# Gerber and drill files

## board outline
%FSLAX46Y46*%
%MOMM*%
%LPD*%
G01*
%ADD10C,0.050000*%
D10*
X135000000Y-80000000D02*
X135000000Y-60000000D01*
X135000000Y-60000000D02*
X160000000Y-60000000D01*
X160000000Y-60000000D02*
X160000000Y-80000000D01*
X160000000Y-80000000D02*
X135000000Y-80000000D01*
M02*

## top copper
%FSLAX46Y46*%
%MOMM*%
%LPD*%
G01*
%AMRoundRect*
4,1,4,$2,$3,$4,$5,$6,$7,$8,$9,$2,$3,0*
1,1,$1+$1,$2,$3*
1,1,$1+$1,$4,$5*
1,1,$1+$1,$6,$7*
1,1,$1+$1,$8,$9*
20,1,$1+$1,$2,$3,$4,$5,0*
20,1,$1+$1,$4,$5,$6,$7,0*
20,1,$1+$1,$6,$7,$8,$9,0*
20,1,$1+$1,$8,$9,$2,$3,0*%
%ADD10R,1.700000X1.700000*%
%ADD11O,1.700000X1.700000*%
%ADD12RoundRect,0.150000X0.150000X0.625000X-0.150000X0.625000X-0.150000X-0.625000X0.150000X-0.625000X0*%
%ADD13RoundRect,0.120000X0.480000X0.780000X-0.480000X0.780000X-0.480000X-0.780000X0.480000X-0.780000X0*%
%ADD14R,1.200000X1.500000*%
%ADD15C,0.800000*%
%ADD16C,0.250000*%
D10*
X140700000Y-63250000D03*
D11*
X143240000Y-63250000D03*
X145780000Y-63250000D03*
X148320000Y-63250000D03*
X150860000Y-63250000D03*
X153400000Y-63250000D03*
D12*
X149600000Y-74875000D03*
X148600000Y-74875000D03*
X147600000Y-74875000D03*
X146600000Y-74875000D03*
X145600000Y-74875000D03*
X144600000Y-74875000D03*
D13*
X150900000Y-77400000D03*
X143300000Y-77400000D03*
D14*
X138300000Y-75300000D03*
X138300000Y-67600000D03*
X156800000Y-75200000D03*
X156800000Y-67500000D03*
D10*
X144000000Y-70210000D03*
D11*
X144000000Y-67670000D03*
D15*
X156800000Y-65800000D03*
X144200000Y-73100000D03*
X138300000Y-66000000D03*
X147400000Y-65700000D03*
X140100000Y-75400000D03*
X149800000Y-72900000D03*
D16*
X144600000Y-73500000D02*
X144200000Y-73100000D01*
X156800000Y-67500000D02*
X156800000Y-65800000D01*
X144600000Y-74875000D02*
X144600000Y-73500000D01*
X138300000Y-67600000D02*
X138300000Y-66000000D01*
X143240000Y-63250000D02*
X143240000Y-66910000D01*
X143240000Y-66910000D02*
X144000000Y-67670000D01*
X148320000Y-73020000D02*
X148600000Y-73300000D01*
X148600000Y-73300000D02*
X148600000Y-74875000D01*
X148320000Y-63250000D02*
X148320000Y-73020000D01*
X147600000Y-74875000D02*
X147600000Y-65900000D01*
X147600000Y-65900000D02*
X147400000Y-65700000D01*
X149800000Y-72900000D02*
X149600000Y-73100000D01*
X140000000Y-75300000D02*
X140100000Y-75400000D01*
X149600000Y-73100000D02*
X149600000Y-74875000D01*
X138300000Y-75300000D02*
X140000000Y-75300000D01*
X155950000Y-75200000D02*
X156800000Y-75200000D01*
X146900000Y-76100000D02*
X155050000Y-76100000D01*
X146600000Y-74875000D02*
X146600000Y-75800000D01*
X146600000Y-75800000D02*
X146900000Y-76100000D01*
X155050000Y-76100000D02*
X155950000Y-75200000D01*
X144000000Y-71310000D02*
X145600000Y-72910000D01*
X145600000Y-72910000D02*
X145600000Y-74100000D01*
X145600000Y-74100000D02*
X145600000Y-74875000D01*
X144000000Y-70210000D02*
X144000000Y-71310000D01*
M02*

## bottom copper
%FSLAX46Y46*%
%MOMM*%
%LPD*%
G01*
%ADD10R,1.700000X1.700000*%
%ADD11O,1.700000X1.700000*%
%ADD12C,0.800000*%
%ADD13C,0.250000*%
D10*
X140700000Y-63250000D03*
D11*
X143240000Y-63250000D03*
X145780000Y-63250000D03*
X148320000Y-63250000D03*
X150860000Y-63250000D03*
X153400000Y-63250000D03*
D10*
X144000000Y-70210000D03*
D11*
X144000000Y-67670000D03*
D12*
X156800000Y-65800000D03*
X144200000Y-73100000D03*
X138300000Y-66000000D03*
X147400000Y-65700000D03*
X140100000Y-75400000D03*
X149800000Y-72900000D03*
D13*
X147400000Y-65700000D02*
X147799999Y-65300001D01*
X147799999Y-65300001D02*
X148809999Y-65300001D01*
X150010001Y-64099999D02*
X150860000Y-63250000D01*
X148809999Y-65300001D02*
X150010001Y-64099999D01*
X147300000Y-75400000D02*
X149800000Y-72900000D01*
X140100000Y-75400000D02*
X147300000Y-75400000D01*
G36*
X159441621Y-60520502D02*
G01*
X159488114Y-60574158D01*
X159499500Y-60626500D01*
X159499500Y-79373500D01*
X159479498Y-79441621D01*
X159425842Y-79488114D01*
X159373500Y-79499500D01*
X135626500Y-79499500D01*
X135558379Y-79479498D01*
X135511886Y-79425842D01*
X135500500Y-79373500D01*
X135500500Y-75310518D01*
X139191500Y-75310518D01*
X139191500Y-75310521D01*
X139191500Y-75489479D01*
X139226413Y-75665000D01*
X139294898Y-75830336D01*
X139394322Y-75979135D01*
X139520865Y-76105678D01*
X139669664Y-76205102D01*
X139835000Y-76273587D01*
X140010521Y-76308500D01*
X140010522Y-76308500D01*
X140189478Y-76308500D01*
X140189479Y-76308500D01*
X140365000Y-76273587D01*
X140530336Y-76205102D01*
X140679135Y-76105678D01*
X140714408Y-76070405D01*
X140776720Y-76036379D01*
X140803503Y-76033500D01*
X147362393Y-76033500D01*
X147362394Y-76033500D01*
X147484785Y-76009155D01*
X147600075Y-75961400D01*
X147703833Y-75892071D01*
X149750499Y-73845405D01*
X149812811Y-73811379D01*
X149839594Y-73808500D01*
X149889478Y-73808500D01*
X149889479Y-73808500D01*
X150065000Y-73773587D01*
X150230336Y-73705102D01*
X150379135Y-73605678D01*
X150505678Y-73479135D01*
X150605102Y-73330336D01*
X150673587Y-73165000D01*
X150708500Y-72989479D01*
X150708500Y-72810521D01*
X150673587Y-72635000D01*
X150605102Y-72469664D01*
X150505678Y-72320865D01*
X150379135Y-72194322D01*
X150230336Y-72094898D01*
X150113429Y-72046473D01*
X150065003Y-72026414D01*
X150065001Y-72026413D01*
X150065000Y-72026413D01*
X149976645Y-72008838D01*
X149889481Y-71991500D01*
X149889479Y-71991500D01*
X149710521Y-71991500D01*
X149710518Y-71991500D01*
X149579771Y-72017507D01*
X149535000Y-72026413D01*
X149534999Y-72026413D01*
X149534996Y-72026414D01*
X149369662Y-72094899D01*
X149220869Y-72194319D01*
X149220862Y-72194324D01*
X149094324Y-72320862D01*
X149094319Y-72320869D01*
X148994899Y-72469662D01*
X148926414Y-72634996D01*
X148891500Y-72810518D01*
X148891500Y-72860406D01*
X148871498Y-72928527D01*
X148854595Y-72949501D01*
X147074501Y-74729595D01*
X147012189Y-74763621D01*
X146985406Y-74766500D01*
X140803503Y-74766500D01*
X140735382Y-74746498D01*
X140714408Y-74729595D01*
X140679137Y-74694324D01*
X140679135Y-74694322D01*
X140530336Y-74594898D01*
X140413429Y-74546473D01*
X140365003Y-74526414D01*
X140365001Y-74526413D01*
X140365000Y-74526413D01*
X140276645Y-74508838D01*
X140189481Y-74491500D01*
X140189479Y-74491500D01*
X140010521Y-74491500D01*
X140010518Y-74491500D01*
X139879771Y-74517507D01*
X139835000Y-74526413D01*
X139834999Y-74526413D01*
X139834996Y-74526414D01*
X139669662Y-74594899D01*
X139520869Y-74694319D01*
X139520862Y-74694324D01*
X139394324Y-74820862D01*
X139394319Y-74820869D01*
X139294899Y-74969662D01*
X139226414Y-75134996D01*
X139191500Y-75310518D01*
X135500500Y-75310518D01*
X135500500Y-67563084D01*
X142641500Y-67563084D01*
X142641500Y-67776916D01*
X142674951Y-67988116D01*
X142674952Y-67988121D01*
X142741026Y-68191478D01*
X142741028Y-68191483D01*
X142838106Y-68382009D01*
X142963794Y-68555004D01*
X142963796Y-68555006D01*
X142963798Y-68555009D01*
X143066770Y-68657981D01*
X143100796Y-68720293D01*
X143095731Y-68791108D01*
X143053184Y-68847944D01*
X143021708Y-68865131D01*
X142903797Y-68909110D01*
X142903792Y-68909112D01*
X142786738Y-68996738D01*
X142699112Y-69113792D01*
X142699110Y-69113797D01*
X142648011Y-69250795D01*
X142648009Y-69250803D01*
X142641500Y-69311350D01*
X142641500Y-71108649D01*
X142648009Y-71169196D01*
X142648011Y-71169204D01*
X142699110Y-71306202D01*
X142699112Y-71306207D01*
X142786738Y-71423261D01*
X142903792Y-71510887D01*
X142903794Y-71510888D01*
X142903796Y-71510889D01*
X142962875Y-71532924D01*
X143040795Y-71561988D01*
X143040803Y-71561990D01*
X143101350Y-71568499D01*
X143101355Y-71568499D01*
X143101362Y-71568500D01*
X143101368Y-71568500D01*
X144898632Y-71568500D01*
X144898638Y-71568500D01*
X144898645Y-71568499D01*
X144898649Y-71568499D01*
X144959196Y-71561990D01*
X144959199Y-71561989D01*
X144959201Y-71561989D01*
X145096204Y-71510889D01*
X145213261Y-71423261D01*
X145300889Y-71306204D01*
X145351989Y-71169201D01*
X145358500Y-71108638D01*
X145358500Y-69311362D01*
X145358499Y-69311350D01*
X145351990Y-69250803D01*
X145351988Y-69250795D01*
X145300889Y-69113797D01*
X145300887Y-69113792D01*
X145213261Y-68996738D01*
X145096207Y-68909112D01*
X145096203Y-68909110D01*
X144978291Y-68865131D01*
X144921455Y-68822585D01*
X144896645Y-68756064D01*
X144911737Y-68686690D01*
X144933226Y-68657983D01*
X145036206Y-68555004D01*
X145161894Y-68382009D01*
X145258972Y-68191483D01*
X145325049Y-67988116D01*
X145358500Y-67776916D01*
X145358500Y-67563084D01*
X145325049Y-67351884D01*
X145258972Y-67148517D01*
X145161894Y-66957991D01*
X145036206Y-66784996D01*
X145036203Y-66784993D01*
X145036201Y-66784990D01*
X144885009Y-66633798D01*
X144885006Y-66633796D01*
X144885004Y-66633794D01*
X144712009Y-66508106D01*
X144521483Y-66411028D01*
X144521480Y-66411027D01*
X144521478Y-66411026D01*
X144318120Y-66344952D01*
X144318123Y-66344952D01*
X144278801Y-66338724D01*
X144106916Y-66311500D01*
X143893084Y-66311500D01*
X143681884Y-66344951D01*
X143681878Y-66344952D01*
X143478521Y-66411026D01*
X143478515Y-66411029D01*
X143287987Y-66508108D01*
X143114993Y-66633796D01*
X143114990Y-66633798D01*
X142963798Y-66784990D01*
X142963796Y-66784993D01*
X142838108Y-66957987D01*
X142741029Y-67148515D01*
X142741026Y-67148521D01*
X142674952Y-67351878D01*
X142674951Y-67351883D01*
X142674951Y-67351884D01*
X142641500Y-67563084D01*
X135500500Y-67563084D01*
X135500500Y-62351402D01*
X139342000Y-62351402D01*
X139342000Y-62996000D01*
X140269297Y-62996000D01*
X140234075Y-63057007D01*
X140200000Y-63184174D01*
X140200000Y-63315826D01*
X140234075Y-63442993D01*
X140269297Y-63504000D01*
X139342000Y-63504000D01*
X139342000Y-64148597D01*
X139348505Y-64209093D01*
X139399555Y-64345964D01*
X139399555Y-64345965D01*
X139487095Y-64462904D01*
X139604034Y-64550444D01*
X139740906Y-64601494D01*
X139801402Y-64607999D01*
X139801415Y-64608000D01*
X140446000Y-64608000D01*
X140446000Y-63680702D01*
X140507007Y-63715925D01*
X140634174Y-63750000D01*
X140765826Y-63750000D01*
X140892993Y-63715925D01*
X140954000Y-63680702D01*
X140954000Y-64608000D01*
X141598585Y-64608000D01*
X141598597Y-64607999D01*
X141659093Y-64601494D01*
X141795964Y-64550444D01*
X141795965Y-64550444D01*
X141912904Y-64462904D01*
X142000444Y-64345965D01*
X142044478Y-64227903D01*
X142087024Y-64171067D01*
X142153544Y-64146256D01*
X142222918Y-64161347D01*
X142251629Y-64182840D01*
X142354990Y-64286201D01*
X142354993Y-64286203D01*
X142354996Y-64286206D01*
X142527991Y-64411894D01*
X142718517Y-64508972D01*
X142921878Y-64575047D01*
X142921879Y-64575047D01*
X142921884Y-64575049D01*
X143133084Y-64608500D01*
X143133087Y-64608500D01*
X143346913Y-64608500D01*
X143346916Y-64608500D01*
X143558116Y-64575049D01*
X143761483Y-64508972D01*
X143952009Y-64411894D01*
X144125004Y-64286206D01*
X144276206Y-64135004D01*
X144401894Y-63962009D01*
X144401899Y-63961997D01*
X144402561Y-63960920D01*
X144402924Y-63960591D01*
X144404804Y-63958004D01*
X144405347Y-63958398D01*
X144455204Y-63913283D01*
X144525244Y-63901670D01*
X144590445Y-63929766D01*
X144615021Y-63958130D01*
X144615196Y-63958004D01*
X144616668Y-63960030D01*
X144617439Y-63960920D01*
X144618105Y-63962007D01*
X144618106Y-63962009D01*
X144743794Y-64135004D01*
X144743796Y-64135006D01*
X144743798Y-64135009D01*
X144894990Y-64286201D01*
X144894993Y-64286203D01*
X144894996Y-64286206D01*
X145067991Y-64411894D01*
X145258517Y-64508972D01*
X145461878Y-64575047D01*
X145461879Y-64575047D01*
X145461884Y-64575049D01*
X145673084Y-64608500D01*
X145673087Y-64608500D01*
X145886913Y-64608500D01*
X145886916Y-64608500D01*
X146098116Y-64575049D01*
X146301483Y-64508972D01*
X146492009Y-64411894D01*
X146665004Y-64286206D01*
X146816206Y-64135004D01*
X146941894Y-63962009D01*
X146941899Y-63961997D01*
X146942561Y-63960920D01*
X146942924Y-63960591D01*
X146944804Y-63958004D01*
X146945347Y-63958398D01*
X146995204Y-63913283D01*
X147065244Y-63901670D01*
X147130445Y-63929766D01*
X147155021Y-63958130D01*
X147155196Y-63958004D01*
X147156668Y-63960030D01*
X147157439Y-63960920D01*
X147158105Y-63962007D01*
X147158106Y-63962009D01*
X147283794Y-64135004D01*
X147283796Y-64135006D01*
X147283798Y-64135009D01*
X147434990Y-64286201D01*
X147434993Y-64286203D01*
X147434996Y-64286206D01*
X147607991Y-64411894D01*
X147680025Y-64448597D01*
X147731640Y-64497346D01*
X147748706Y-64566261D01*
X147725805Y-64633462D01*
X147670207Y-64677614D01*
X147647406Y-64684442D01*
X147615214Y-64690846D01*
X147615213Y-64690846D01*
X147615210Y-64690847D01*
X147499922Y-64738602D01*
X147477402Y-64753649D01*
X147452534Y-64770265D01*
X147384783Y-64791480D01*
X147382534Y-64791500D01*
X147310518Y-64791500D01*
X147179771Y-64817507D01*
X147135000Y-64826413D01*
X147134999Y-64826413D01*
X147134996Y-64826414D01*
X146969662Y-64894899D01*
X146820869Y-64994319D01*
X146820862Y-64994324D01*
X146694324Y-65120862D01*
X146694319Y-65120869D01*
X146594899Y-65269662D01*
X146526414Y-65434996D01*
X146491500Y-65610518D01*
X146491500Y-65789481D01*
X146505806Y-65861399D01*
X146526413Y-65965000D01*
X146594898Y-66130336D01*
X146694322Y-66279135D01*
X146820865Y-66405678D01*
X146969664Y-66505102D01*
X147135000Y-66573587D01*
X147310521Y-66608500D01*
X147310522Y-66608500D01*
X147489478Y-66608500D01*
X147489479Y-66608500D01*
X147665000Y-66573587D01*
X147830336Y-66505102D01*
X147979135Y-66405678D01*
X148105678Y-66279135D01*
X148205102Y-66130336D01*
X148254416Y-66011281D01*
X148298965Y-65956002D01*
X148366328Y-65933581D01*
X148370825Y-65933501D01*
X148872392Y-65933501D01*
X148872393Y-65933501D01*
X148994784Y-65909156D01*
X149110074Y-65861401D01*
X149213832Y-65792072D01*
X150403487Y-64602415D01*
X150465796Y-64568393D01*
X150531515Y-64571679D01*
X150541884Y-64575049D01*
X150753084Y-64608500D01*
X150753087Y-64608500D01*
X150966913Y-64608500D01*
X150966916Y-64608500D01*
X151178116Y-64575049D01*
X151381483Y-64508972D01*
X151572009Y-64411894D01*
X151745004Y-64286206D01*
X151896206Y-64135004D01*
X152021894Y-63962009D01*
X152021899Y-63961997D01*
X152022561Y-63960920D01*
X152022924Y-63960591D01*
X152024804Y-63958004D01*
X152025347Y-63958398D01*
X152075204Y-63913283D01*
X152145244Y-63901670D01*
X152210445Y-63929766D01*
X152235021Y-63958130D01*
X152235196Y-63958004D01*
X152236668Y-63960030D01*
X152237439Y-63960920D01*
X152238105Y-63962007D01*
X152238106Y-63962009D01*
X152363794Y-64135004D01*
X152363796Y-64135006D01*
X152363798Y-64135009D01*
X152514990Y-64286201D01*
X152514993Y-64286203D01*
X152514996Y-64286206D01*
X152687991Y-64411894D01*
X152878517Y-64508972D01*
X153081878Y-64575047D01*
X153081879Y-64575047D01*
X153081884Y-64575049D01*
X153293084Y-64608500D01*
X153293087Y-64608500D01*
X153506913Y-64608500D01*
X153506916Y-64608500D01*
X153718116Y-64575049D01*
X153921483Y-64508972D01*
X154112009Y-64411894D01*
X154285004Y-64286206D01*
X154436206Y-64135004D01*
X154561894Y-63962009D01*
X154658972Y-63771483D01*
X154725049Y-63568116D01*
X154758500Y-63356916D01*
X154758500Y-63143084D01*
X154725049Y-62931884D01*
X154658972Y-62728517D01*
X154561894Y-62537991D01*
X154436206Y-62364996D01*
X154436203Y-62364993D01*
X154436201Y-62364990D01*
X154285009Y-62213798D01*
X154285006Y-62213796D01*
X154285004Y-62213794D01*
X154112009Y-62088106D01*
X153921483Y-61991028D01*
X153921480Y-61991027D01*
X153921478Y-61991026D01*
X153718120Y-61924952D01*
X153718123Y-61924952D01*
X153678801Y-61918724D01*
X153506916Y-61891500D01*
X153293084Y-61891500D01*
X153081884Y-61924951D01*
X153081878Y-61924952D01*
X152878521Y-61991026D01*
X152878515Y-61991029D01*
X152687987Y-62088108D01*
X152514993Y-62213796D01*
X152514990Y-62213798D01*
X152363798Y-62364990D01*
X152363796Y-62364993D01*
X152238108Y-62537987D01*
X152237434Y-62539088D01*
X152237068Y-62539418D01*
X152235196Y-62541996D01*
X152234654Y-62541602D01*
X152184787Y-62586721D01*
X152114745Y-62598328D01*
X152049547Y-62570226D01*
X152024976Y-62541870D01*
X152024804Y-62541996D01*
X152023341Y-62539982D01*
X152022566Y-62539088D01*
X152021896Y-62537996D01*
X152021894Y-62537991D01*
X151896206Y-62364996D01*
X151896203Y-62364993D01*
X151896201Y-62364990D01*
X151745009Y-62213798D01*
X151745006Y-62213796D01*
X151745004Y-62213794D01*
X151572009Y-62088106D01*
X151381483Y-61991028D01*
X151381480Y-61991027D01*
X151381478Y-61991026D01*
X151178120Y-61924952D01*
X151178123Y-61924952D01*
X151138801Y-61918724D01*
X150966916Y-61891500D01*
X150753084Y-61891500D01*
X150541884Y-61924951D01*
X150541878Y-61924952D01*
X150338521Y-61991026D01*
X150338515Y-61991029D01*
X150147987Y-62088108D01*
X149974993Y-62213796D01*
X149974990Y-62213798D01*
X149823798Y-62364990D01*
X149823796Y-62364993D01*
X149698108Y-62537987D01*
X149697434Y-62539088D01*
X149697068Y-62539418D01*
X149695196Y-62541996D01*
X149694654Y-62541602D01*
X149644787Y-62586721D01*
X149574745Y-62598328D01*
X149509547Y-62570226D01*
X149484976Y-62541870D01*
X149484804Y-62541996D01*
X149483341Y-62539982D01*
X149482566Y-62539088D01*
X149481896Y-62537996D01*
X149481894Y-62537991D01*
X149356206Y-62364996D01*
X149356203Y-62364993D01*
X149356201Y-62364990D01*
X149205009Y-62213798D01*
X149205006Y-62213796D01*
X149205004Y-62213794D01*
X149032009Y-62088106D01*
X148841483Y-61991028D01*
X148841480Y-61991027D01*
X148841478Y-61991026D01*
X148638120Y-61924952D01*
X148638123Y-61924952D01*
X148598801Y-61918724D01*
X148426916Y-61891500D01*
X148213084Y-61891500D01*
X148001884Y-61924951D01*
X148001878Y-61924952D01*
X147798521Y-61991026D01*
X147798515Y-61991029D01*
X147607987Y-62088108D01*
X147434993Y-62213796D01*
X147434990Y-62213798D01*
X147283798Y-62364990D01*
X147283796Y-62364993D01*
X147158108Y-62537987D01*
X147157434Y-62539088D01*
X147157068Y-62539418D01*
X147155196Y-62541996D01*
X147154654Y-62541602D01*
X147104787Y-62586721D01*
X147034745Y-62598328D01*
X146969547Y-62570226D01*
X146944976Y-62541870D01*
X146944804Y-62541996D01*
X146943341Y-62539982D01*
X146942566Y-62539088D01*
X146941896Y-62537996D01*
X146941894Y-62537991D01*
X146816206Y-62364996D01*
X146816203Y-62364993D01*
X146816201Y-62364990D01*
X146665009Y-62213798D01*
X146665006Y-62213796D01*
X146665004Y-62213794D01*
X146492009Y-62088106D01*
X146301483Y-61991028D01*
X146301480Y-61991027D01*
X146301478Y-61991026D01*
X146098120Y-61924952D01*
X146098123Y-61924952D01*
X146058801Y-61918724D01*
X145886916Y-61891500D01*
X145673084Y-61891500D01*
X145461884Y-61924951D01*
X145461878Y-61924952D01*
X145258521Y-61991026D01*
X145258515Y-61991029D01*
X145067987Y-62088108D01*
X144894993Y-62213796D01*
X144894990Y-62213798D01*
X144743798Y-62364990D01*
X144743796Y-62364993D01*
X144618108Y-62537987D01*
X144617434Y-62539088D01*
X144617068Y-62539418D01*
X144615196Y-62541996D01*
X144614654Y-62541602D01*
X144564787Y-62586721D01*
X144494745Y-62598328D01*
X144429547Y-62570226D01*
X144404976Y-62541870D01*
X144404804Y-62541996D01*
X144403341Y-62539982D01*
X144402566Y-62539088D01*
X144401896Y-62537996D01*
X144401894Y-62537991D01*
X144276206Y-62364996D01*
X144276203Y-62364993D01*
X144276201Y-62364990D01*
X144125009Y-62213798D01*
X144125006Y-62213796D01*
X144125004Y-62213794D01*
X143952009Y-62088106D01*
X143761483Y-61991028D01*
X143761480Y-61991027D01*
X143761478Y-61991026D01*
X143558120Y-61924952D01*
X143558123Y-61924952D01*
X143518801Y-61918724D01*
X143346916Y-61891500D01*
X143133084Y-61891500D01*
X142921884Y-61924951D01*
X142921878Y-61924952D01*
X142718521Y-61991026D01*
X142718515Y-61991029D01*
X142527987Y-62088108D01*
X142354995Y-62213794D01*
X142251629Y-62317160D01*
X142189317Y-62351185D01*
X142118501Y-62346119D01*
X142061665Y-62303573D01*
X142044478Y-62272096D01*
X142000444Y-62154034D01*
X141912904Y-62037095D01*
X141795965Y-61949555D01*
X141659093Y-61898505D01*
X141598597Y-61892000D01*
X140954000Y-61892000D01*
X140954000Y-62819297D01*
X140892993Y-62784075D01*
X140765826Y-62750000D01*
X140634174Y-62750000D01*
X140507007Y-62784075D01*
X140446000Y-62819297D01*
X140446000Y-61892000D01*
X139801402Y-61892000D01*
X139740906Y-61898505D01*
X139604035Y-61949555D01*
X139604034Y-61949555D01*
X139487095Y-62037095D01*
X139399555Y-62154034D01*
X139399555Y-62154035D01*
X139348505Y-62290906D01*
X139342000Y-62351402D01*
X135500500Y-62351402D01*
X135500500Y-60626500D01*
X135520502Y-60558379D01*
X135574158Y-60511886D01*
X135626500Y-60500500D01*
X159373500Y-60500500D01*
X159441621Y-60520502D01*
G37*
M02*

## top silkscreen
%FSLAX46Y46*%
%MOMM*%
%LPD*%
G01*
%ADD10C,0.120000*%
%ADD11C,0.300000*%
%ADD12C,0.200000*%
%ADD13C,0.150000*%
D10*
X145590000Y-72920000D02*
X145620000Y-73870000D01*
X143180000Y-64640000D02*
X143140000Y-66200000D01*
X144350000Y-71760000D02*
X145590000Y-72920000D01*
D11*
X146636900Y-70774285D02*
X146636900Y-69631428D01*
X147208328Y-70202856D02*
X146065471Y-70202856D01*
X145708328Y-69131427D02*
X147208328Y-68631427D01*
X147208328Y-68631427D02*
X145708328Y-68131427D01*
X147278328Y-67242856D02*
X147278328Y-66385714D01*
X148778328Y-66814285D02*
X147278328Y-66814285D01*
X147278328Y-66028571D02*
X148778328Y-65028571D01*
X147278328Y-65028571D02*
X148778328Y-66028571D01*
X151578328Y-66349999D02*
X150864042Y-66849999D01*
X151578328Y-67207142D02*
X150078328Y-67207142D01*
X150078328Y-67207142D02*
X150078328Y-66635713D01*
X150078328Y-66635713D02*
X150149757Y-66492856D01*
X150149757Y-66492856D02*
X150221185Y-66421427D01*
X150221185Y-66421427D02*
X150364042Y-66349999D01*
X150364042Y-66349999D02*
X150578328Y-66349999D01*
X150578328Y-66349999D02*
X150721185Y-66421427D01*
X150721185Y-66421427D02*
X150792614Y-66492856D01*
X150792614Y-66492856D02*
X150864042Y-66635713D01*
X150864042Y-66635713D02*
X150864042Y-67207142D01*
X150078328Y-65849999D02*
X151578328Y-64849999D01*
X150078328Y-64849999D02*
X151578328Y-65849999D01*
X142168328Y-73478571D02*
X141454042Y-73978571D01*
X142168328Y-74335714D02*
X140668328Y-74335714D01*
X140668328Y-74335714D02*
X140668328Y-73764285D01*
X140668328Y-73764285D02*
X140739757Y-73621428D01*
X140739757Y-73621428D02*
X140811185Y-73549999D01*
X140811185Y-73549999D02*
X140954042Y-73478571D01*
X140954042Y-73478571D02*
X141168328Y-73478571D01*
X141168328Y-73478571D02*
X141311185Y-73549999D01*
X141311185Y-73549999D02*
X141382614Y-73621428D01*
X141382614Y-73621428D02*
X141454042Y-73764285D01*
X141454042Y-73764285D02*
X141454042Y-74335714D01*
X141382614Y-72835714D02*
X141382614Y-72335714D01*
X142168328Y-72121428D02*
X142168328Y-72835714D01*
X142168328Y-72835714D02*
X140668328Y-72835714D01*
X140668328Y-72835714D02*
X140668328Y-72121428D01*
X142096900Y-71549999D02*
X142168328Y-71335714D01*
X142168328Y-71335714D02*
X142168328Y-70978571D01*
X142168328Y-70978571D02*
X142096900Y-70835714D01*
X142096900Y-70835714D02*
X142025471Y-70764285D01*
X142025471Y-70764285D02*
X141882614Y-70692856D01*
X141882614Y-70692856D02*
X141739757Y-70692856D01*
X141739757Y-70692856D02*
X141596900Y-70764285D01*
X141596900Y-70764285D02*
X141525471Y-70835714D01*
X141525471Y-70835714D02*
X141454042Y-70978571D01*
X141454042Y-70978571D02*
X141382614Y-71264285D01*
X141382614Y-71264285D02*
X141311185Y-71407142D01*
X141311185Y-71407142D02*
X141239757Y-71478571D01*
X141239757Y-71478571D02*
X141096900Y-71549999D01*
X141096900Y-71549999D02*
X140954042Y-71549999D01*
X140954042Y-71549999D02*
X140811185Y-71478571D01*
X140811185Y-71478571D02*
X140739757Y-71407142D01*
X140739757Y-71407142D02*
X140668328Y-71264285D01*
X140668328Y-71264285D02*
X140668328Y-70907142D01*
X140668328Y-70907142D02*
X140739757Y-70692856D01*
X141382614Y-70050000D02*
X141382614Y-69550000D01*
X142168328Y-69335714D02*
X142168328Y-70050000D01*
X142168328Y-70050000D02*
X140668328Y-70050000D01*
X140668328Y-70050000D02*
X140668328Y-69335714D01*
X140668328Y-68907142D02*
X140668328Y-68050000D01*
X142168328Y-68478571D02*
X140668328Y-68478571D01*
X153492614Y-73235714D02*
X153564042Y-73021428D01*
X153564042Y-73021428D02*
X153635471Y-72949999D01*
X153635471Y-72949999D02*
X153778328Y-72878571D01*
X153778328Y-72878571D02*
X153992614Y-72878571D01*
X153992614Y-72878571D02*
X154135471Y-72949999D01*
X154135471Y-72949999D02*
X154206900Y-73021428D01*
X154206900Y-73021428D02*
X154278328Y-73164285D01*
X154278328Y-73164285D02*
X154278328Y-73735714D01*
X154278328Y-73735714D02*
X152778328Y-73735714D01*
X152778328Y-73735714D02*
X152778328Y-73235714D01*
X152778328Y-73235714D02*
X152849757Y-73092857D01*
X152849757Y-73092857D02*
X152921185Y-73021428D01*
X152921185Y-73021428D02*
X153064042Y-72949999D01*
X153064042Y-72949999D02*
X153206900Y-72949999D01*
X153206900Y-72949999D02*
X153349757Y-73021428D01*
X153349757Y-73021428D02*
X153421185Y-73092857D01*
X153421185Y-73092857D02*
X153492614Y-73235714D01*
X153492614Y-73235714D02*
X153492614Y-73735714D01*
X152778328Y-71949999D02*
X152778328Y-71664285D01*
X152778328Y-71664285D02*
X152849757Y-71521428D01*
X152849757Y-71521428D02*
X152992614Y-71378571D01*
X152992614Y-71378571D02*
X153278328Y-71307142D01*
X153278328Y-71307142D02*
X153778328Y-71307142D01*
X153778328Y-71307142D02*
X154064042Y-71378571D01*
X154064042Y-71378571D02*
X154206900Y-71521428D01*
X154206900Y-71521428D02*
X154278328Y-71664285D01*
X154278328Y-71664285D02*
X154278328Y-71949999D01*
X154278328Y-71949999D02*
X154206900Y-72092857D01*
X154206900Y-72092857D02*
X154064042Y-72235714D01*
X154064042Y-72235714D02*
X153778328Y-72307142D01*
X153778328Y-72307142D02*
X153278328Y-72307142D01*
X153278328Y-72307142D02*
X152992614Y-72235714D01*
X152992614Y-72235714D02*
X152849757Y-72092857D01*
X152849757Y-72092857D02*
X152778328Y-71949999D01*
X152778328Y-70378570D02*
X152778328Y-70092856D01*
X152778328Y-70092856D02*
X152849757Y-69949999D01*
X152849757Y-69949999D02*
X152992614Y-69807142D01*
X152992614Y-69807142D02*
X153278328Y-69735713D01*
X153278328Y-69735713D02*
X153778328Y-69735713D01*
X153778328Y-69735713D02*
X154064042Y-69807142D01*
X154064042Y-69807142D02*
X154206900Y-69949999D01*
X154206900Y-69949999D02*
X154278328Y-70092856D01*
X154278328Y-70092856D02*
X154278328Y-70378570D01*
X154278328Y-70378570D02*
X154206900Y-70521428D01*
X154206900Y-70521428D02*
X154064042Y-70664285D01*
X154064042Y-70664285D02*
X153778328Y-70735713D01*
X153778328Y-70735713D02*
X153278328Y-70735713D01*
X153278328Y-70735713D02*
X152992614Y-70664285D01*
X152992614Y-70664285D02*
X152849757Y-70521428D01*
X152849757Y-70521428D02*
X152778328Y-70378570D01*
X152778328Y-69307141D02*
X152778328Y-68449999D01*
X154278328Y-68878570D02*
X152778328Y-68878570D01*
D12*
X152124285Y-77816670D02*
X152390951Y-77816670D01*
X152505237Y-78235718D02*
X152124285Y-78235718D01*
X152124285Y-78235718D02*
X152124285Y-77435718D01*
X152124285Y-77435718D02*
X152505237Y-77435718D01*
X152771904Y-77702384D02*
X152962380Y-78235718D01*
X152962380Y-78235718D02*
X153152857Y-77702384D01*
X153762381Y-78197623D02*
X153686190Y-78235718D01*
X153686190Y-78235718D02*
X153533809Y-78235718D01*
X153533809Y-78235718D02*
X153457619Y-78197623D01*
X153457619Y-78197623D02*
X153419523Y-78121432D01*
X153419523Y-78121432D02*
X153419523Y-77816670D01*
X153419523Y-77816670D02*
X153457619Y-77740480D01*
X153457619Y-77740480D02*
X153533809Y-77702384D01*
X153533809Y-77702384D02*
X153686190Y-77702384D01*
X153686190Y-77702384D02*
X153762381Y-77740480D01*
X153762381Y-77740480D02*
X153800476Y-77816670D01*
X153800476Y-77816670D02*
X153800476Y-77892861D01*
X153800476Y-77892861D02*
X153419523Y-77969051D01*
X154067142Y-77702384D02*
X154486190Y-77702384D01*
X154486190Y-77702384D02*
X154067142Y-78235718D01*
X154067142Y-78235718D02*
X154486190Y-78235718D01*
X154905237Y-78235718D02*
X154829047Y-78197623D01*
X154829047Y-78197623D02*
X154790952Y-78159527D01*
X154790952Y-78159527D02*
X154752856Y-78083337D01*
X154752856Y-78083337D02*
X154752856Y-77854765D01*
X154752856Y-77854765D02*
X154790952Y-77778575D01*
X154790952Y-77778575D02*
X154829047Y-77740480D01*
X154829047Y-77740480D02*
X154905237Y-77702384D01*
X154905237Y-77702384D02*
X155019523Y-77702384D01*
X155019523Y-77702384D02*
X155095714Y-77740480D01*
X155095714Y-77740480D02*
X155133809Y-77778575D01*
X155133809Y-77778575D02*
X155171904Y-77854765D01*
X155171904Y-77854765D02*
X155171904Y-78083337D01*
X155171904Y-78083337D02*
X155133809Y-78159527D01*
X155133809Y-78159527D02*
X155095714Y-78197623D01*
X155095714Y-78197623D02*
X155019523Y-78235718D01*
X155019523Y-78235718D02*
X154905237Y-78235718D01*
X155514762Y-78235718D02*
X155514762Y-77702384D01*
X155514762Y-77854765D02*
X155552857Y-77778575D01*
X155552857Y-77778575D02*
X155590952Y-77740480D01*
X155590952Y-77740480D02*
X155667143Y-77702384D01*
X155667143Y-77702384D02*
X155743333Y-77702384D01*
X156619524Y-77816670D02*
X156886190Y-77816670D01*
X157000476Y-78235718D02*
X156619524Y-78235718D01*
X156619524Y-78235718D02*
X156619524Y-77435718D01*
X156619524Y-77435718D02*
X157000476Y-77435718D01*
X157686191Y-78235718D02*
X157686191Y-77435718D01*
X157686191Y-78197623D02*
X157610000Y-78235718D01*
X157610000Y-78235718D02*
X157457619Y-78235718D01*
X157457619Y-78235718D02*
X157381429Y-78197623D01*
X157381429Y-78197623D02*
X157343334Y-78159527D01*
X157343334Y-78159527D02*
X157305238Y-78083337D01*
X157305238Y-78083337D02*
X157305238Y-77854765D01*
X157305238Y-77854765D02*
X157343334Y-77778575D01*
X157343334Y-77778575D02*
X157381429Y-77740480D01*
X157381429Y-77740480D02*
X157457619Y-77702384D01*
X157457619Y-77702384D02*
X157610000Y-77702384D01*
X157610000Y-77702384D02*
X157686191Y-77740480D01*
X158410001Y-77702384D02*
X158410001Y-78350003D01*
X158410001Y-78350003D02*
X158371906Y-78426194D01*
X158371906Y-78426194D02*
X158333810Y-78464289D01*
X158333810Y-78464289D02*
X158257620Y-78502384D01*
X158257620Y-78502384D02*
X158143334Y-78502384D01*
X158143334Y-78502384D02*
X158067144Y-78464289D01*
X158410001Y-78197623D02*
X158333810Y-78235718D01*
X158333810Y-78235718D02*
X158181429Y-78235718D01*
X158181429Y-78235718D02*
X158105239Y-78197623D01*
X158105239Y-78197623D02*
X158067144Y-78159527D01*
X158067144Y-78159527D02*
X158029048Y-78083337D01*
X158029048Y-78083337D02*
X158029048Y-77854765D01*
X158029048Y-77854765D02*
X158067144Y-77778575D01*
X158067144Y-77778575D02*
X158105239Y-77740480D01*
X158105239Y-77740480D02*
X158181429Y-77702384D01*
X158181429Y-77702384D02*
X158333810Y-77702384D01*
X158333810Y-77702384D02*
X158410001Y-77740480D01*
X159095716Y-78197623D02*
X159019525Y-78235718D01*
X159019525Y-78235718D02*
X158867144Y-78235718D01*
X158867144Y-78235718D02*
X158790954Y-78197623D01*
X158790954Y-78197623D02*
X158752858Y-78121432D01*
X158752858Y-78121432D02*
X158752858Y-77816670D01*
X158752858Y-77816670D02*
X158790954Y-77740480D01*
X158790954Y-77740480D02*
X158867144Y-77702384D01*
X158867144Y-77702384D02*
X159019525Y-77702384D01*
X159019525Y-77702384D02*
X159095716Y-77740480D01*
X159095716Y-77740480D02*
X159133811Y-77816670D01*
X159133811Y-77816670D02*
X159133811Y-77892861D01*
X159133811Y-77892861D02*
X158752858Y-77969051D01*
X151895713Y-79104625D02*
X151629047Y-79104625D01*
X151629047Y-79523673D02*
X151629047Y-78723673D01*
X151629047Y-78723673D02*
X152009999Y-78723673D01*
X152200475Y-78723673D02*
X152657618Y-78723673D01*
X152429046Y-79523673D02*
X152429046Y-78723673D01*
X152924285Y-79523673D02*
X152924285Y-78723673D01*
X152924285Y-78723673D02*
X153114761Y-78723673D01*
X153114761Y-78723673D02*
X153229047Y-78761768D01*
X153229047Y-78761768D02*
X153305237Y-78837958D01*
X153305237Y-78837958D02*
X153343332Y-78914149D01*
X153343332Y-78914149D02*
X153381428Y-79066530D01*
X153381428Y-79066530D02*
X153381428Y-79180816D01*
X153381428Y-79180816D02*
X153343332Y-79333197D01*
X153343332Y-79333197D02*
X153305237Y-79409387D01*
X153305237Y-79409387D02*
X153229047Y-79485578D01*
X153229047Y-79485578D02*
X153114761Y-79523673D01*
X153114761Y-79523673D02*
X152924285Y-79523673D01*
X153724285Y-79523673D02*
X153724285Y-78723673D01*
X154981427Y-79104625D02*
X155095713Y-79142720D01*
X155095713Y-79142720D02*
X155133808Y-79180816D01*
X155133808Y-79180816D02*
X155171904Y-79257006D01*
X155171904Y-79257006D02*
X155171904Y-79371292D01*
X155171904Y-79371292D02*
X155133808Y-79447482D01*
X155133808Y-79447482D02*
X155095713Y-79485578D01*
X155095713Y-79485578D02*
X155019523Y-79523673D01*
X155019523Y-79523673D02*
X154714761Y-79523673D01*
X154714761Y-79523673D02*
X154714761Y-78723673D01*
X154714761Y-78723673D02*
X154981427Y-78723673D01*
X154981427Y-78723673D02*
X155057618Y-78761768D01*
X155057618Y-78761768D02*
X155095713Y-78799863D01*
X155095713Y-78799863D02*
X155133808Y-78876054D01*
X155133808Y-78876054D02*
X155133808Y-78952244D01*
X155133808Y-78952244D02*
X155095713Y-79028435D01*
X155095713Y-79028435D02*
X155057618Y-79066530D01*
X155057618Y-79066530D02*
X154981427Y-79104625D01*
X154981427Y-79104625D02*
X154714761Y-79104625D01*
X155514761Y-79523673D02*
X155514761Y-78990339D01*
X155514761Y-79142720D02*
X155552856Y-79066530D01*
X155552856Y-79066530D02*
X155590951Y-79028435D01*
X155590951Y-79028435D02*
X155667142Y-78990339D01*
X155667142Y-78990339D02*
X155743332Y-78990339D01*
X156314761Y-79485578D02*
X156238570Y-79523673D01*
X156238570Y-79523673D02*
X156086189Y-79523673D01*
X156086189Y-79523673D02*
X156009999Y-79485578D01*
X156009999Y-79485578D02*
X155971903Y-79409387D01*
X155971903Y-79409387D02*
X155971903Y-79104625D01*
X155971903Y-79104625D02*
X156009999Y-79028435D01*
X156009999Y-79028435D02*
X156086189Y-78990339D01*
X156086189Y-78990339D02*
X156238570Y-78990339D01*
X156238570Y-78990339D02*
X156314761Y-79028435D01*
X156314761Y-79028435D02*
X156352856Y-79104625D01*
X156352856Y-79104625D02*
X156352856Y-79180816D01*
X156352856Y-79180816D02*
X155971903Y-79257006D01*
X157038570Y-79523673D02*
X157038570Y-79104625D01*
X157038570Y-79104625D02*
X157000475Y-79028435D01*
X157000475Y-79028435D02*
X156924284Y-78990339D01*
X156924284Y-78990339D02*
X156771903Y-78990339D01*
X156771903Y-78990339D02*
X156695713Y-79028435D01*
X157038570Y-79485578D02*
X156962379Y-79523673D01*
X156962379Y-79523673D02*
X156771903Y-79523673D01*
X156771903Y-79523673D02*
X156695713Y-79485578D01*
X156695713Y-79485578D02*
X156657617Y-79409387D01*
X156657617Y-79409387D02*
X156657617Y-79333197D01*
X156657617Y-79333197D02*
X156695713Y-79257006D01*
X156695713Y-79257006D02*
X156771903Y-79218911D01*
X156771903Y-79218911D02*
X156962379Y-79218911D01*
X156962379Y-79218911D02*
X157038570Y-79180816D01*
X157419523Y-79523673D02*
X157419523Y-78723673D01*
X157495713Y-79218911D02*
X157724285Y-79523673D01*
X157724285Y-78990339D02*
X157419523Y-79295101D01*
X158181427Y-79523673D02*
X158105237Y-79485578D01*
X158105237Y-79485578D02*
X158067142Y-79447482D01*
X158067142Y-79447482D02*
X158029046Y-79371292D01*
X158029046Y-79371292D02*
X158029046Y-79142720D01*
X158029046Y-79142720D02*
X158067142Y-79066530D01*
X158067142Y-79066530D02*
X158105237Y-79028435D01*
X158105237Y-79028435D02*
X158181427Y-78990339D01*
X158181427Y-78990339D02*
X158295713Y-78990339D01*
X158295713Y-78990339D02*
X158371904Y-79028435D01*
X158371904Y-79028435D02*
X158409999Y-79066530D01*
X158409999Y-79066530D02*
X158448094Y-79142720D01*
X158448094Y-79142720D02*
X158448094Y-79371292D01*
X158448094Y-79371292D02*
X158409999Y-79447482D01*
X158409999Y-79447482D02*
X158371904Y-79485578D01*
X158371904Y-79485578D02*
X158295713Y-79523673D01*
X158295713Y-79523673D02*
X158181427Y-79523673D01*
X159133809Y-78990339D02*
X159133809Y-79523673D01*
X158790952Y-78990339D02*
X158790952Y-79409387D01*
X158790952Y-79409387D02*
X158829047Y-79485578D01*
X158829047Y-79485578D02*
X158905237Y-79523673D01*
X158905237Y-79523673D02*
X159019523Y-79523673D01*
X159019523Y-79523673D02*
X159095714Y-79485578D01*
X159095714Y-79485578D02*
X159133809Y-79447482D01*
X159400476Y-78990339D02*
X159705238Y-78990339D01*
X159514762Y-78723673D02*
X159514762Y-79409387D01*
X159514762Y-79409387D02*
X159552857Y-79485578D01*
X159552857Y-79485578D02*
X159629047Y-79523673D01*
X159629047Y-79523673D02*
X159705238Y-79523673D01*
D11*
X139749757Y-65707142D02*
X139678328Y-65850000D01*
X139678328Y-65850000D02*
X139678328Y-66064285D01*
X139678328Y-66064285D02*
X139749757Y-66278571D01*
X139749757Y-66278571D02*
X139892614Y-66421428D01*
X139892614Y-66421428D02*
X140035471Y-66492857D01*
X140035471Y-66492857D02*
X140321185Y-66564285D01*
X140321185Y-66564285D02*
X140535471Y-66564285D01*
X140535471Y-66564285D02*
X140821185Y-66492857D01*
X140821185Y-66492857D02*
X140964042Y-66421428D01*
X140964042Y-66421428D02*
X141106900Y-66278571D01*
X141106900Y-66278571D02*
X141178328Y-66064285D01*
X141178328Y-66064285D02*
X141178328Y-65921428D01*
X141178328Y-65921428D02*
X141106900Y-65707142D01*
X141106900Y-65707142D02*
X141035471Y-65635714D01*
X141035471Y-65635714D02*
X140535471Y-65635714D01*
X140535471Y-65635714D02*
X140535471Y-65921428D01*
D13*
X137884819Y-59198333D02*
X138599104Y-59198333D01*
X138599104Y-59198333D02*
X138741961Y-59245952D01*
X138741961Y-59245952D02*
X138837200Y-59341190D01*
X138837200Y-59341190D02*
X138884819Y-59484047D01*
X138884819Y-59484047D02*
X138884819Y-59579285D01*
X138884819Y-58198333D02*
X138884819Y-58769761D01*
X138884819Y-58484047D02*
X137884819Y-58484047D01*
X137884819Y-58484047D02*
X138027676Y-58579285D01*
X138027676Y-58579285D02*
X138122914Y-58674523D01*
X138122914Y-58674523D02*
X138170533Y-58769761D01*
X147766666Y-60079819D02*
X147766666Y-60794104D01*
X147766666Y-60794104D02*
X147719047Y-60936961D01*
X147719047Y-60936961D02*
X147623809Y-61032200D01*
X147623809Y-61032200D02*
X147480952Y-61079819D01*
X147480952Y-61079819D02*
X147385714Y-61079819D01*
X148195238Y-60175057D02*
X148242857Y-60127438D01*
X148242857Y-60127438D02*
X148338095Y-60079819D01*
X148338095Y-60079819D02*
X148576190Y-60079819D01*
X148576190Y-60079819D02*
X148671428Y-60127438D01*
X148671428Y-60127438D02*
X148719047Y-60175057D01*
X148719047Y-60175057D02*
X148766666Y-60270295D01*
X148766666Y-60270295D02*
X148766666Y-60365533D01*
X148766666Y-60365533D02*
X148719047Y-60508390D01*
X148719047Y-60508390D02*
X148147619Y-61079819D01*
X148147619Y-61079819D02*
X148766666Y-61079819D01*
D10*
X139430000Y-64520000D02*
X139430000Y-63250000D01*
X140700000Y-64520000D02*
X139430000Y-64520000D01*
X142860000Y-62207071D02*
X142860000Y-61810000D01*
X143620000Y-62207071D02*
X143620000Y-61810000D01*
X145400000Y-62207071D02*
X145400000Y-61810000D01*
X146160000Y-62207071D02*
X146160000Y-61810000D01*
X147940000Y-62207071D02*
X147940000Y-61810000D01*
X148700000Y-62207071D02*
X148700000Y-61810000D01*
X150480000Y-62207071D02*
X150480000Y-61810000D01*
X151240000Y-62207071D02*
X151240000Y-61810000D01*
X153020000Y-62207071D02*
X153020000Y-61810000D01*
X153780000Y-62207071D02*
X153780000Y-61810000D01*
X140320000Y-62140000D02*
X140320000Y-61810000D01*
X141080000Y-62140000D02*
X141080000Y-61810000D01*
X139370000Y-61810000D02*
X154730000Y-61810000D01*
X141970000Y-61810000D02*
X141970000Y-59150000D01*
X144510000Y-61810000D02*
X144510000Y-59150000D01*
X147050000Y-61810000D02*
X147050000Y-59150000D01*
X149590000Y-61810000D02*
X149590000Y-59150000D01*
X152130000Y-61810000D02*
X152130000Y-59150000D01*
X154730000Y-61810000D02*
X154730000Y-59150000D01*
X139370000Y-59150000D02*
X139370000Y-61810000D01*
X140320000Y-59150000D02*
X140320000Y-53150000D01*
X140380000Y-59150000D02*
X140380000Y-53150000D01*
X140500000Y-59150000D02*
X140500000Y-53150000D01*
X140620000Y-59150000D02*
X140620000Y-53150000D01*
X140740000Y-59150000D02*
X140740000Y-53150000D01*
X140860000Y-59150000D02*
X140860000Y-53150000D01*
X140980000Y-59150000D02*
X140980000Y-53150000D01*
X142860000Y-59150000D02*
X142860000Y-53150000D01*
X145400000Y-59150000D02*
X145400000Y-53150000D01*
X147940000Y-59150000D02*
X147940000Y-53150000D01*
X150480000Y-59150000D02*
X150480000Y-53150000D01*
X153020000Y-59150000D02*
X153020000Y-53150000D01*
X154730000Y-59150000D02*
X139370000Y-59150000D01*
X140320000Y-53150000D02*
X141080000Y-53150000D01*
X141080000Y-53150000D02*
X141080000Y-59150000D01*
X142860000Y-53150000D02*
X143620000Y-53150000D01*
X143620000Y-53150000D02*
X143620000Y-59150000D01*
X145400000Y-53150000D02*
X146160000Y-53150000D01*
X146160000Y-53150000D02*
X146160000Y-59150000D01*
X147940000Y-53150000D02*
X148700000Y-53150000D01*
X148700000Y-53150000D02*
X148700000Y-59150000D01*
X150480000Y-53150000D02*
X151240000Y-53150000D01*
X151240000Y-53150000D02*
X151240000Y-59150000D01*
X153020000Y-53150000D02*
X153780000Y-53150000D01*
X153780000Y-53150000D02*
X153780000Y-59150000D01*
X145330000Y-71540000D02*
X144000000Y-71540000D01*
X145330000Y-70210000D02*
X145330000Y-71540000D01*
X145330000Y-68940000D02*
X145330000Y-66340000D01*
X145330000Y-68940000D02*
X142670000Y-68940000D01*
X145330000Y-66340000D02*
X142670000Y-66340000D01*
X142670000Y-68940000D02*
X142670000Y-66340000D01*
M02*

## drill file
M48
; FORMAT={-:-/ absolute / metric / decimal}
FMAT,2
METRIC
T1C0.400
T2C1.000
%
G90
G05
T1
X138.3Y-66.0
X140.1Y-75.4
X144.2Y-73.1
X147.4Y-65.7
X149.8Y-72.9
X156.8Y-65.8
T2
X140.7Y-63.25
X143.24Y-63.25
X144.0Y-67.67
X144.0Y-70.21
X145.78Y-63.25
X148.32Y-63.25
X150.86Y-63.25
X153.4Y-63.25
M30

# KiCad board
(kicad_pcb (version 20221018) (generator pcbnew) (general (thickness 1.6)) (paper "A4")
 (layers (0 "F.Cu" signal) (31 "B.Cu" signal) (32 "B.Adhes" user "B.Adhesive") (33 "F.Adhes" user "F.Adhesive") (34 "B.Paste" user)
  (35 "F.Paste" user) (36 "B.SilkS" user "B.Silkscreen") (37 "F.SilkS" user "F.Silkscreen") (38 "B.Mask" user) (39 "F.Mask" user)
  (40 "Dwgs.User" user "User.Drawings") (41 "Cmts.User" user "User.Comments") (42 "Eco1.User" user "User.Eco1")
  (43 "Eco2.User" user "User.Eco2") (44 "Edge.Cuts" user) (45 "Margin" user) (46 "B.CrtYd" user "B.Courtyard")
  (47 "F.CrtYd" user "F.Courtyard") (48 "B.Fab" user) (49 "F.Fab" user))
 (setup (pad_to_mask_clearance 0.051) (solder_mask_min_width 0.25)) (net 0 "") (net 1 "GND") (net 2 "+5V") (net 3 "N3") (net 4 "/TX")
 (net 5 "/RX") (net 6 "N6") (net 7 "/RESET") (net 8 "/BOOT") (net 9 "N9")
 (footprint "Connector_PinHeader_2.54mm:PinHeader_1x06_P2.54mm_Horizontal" (layer "F.Cu") (at 140.7 63.25 90)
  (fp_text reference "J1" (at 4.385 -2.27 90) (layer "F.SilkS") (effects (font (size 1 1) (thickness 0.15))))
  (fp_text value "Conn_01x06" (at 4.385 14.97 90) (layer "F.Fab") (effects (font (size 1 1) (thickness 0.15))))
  (fp_line (start -1.27 -1.27) (end 0 -1.27) (stroke (width 0.12) (type solid)) (layer "F.SilkS"))
  (fp_line (start -1.27 0) (end -1.27 -1.27) (stroke (width 0.12) (type solid)) (layer "F.SilkS"))
  (fp_line (start 1.042929 2.16) (end 1.44 2.16) (stroke (width 0.12) (type solid)) (layer "F.SilkS"))
  (fp_line (start 1.042929 2.92) (end 1.44 2.92) (stroke (width 0.12) (type solid)) (layer "F.SilkS"))
  (fp_line (start 1.042929 4.7) (end 1.44 4.7) (stroke (width 0.12) (type solid)) (layer "F.SilkS"))
  (fp_line (start 1.042929 5.46) (end 1.44 5.46) (stroke (width 0.12) (type solid)) (layer "F.SilkS"))
  (fp_line (start 1.042929 7.24) (end 1.44 7.24) (stroke (width 0.12) (type solid)) (layer "F.SilkS"))
  (fp_line (start 1.042929 8) (end 1.44 8) (stroke (width 0.12) (type solid)) (layer "F.SilkS"))
  (fp_line (start 1.042929 9.78) (end 1.44 9.78) (stroke (width 0.12) (type solid)) (layer "F.SilkS"))
  (fp_line (start 1.042929 10.54) (end 1.44 10.54) (stroke (width 0.12) (type solid)) (layer "F.SilkS"))
  (fp_line (start 1.042929 12.32) (end 1.44 12.32) (stroke (width 0.12) (type solid)) (layer "F.SilkS"))
  (fp_line (start 1.042929 13.08) (end 1.44 13.08) (stroke (width 0.12) (type solid)) (layer "F.SilkS"))
  (fp_line (start 1.11 -0.38) (end 1.44 -0.38) (stroke (width 0.12) (type solid)) (layer "F.SilkS"))
  (fp_line (start 1.11 0.38) (end 1.44 0.38) (stroke (width 0.12) (type solid)) (layer "F.SilkS"))
  (fp_line (start 1.44 -1.33) (end 1.44 14.03) (stroke (width 0.12) (type solid)) (layer "F.SilkS"))
  (fp_line (start 1.44 1.27) (end 4.1 1.27) (stroke (width 0.12) (type solid)) (layer "F.SilkS"))
  (fp_line (start 1.44 3.81) (end 4.1 3.81) (stroke (width 0.12) (type solid)) (layer "F.SilkS"))
  (fp_line (start 1.44 6.35) (end 4.1 6.35) (stroke (width 0.12) (type solid)) (layer "F.SilkS"))
  (fp_line (start 1.44 8.89) (end 4.1 8.89) (stroke (width 0.12) (type solid)) (layer "F.SilkS"))
  (fp_line (start 1.44 11.43) (end 4.1 11.43) (stroke (width 0.12) (type solid)) (layer "F.SilkS"))
  (fp_line (start 1.44 14.03) (end 4.1 14.03) (stroke (width 0.12) (type solid)) (layer "F.SilkS"))
  (fp_line (start 4.1 -1.33) (end 1.44 -1.33) (stroke (width 0.12) (type solid)) (layer "F.SilkS"))
  (fp_line (start 4.1 -0.38) (end 10.1 -0.38) (stroke (width 0.12) (type solid)) (layer "F.SilkS"))
  (fp_line (start 4.1 -0.32) (end 10.1 -0.32) (stroke (width 0.12) (type solid)) (layer "F.SilkS"))
  (fp_line (start 4.1 -0.2) (end 10.1 -0.2) (stroke (width 0.12) (type solid)) (layer "F.SilkS"))
  (fp_line (start 4.1 -0.08) (end 10.1 -0.08) (stroke (width 0.12) (type solid)) (layer "F.SilkS"))
  (fp_line (start 4.1 0.04) (end 10.1 0.04) (stroke (width 0.12) (type solid)) (layer "F.SilkS"))
  (fp_line (start 4.1 0.16) (end 10.1 0.16) (stroke (width 0.12) (type solid)) (layer "F.SilkS"))
  (fp_line (start 4.1 0.28) (end 10.1 0.28) (stroke (width 0.12) (type solid)) (layer "F.SilkS"))
  (fp_line (start 4.1 2.16) (end 10.1 2.16) (stroke (width 0.12) (type solid)) (layer "F.SilkS"))
  (fp_line (start 4.1 4.7) (end 10.1 4.7) (stroke (width 0.12) (type solid)) (layer "F.SilkS"))
  (fp_line (start 4.1 7.24) (end 10.1 7.24) (stroke (width 0.12) (type solid)) (layer "F.SilkS"))
  (fp_line (start 4.1 9.78) (end 10.1 9.78) (stroke (width 0.12) (type solid)) (layer "F.SilkS"))
  (fp_line (start 4.1 12.32) (end 10.1 12.32) (stroke (width 0.12) (type solid)) (layer "F.SilkS"))
  (fp_line (start 4.1 14.03) (end 4.1 -1.33) (stroke (width 0.12) (type solid)) (layer "F.SilkS"))
  (fp_line (start 10.1 -0.38) (end 10.1 0.38) (stroke (width 0.12) (type solid)) (layer "F.SilkS"))
  (fp_line (start 10.1 0.38) (end 4.1 0.38) (stroke (width 0.12) (type solid)) (layer "F.SilkS"))
  (fp_line (start 10.1 2.16) (end 10.1 2.92) (stroke (width 0.12) (type solid)) (layer "F.SilkS"))
  (fp_line (start 10.1 2.92) (end 4.1 2.92) (stroke (width 0.12) (type solid)) (layer "F.SilkS"))
  (fp_line (start 10.1 4.7) (end 10.1 5.46) (stroke (width 0.12) (type solid)) (layer "F.SilkS"))
  (fp_line (start 10.1 5.46) (end 4.1 5.46) (stroke (width 0.12) (type solid)) (layer "F.SilkS"))
  (fp_line (start 10.1 7.24) (end 10.1 8) (stroke (width 0.12) (type solid)) (layer "F.SilkS"))
  (fp_line (start 10.1 8) (end 4.1 8) (stroke (width 0.12) (type solid)) (layer "F.SilkS"))
  (fp_line (start 10.1 9.78) (end 10.1 10.54) (stroke (width 0.12) (type solid)) (layer "F.SilkS"))
  (fp_line (start 10.1 10.54) (end 4.1 10.54) (stroke (width 0.12) (type solid)) (layer "F.SilkS"))
  (fp_line (start 10.1 12.32) (end 10.1 13.08) (stroke (width 0.12) (type solid)) (layer "F.SilkS"))
  (fp_line (start 10.1 13.08) (end 4.1 13.08) (stroke (width 0.12) (type solid)) (layer "F.SilkS"))
  (pad "1" thru_hole rect (at 0 0 90) (size 1.7 1.7) (drill 1) (layers "*.Cu" "*.Mask") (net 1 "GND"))
  (pad "2" thru_hole oval (at 0 2.54 90) (size 1.7 1.7) (drill 1) (layers "*.Cu" "*.Mask") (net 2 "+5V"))
  (pad "3" thru_hole oval (at 0 5.08 90) (size 1.7 1.7) (drill 1) (layers "*.Cu" "*.Mask") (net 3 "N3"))
  (pad "4" thru_hole oval (at 0 7.62 90) (size 1.7 1.7) (drill 1) (layers "*.Cu" "*.Mask") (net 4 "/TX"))
  (pad "5" thru_hole oval (at 0 10.16 90) (size 1.7 1.7) (drill 1) (layers "*.Cu" "*.Mask") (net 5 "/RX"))
  (pad "6" thru_hole oval (at 0 12.7 90) (size 1.7 1.7) (drill 1) (layers "*.Cu" "*.Mask") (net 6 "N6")))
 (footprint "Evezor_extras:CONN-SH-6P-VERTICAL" (layer "F.Cu") (at 147.1 74.875 180)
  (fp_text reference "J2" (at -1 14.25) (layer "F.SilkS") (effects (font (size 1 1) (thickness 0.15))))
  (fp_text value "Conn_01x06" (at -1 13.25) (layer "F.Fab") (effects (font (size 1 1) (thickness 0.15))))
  (pad "1" smd roundrect (at -2.5 0 180) (size 0.6 1.55) (layers "F.Cu" "F.Paste" "F.Mask") (roundrect_rratio 0.25) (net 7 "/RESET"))
  (pad "2" smd roundrect (at -1.5 0 180) (size 0.6 1.55) (layers "F.Cu" "F.Paste" "F.Mask") (roundrect_rratio 0.25) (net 4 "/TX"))
  (pad "3" smd roundrect (at -0.5 0 180) (size 0.6 1.55) (layers "F.Cu" "F.Paste" "F.Mask") (roundrect_rratio 0.25) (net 5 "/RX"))
  (pad "4" smd roundrect (at 0.5 0 180) (size 0.6 1.55) (layers "F.Cu" "F.Paste" "F.Mask") (roundrect_rratio 0.25) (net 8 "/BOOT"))
  (pad "5" smd roundrect (at 1.5 0 180) (size 0.6 1.55) (layers "F.Cu" "F.Paste" "F.Mask") (roundrect_rratio 0.25) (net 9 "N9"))
  (pad "6" smd roundrect (at 2.5 0 180) (size 0.6 1.55) (layers "F.Cu" "F.Paste" "F.Mask") (roundrect_rratio 0.25) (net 1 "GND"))
  (pad "MP" smd roundrect (at -3.8 -2.525 180) (size 1.2 1.8) (layers "F.Cu" "F.Paste" "F.Mask") (roundrect_rratio 0.1))
  (pad "MP" smd roundrect (at 3.8 -2.525 180) (size 1.2 1.8) (layers "F.Cu" "F.Paste" "F.Mask") (roundrect_rratio 0.1)))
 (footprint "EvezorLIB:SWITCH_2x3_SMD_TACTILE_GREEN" (layer "F.Cu") (at 138.3 71.45 90)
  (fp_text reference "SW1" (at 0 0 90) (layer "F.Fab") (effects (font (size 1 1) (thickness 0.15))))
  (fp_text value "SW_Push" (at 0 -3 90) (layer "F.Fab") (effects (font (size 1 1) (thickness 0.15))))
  (pad "1" smd rect (at -3.85 0 90) (size 1.5 1.2) (layers "F.Cu" "F.Paste" "F.Mask") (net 7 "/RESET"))
  (pad "2" smd rect (at 3.85 0 90) (size 1.5 1.2) (layers "F.Cu" "F.Paste" "F.Mask") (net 1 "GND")))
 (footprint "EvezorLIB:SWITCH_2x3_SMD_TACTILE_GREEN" (layer "F.Cu") (at 156.8 71.35 90)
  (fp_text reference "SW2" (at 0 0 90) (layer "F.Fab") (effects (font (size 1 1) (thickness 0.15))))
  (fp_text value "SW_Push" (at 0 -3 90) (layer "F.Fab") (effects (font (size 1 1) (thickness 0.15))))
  (pad "1" smd rect (at -3.85 0 90) (size 1.5 1.2) (layers "F.Cu" "F.Paste" "F.Mask") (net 8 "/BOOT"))
  (pad "2" smd rect (at 3.85 0 90) (size 1.5 1.2) (layers "F.Cu" "F.Paste" "F.Mask") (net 1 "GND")))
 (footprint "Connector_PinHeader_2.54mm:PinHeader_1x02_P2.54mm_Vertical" (layer "F.Cu") (at 144 70.21 180)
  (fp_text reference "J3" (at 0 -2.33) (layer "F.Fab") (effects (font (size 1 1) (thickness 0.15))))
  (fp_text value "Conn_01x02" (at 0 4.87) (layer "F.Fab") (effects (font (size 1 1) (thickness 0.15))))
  (fp_line (start -1.33 -1.33) (end 0 -1.33) (stroke (width 0.12) (type solid)) (layer "F.SilkS"))
  (fp_line (start -1.33 0) (end -1.33 -1.33) (stroke (width 0.12) (type solid)) (layer "F.SilkS"))
  (fp_line (start -1.33 1.27) (end -1.33 3.87) (stroke (width 0.12) (type solid)) (layer "F.SilkS"))
  (fp_line (start -1.33 1.27) (end 1.33 1.27) (stroke (width 0.12) (type solid)) (layer "F.SilkS"))
  (fp_line (start -1.33 3.87) (end 1.33 3.87) (stroke (width 0.12) (type solid)) (layer "F.SilkS"))
  (fp_line (start 1.33 1.27) (end 1.33 3.87) (stroke (width 0.12) (type solid)) (layer "F.SilkS"))
  (pad "1" thru_hole rect (at 0 0 180) (size 1.7 1.7) (drill 1) (layers "*.Cu" "*.Mask") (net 9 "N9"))
  (pad "2" thru_hole oval (at 0 2.54 180) (size 1.7 1.7) (drill 1) (layers "*.Cu" "*.Mask") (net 2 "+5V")))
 (gr_line (start 145.59 72.92) (end 145.62 73.87) (stroke (width 0.12) (type solid)) (layer "F.SilkS"))
 (gr_line (start 143.18 64.64) (end 143.14 66.2) (stroke (width 0.12) (type solid)) (layer "F.SilkS"))
 (gr_line (start 144.35 71.76) (end 145.59 72.92) (stroke (width 0.12) (type solid)) (layer "F.SilkS"))
 (gr_line (start 135 80) (end 135 60) (stroke (width 0.05) (type solid)) (layer "Edge.Cuts"))
 (gr_line (start 135 60) (end 160 60) (stroke (width 0.05) (type solid)) (layer "Edge.Cuts"))
 (gr_line (start 160 60) (end 160 80) (stroke (width 0.05) (type solid)) (layer "Edge.Cuts"))
 (gr_line (start 160 80) (end 135 80) (stroke (width 0.05) (type solid)) (layer "Edge.Cuts"))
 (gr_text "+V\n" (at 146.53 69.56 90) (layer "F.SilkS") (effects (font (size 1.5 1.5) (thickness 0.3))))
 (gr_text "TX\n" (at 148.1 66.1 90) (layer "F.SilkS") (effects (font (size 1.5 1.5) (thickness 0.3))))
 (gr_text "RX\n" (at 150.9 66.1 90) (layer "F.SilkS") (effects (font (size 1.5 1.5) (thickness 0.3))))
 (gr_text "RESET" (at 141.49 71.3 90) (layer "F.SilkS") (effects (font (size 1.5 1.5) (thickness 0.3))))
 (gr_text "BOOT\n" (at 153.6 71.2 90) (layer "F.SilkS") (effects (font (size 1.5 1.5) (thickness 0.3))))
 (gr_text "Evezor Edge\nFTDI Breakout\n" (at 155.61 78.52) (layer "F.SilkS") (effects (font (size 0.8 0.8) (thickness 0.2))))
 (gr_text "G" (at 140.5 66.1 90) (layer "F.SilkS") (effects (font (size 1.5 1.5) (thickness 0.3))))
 (segment (start 144.6 73.5) (end 144.2 73.1) (width 0.25) (layer "F.Cu") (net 1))
 (segment (start 156.8 67.5) (end 156.8 65.8) (width 0.25) (layer "F.Cu") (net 1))
 (segment (start 144.6 74.875) (end 144.6 73.5) (width 0.25) (layer "F.Cu") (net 1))
 (segment (start 138.3 67.6) (end 138.3 66) (width 0.25) (layer "F.Cu") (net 1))
 (via (at 156.8 65.8) (size 0.8) (drill 0.4) (layers "F.Cu" "B.Cu") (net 1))
 (via (at 144.2 73.1) (size 0.8) (drill 0.4) (layers "F.Cu" "B.Cu") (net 1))
 (via (at 138.3 66) (size 0.8) (drill 0.4) (layers "F.Cu" "B.Cu") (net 1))
 (segment (start 143.24 63.25) (end 143.24 66.91) (width 0.25) (layer "F.Cu") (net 2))
 (segment (start 143.24 66.91) (end 144 67.67) (width 0.25) (layer "F.Cu") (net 2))
 (segment (start 148.32 73.02) (end 148.6 73.3) (width 0.25) (layer "F.Cu") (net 4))
 (segment (start 148.6 73.3) (end 148.6 74.875) (width 0.25) (layer "F.Cu") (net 4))
 (segment (start 148.32 63.25) (end 148.32 73.02) (width 0.25) (layer "F.Cu") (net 4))
 (segment (start 147.6 74.875) (end 147.6 65.9) (width 0.25) (layer "F.Cu") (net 5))
 (segment (start 147.6 65.9) (end 147.4 65.7) (width 0.25) (layer "F.Cu") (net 5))
 (via (at 147.4 65.7) (size 0.8) (drill 0.4) (layers "F.Cu" "B.Cu") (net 5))
 (segment (start 147.4 65.7) (end 147.799999 65.300001) (width 0.25) (layer "B.Cu") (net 5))
 (segment (start 147.799999 65.300001) (end 148.809999 65.300001) (width 0.25) (layer "B.Cu") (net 5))
 (segment (start 150.010001 64.099999) (end 150.86 63.25) (width 0.25) (layer "B.Cu") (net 5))
 (segment (start 148.809999 65.300001) (end 150.010001 64.099999) (width 0.25) (layer "B.Cu") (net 5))
 (segment (start 149.8 72.9) (end 149.6 73.1) (width 0.25) (layer "F.Cu") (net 7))
 (segment (start 140 75.3) (end 140.1 75.4) (width 0.25) (layer "F.Cu") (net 7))
 (segment (start 149.6 73.1) (end 149.6 74.875) (width 0.25) (layer "F.Cu") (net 7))
 (segment (start 138.3 75.3) (end 140 75.3) (width 0.25) (layer "F.Cu") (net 7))
 (via (at 140.1 75.4) (size 0.8) (drill 0.4) (layers "F.Cu" "B.Cu") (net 7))
 (via (at 149.8 72.9) (size 0.8) (drill 0.4) (layers "F.Cu" "B.Cu") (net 7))
 (segment (start 147.3 75.4) (end 149.8 72.9) (width 0.25) (layer "B.Cu") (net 7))
 (segment (start 140.1 75.4) (end 147.3 75.4) (width 0.25) (layer "B.Cu") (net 7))
 (segment (start 155.95 75.2) (end 156.8 75.2) (width 0.25) (layer "F.Cu") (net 8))
 (segment (start 146.9 76.1) (end 155.05 76.1) (width 0.25) (layer "F.Cu") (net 8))
 (segment (start 146.6 74.875) (end 146.6 75.8) (width 0.25) (layer "F.Cu") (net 8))
 (segment (start 146.6 75.8) (end 146.9 76.1) (width 0.25) (layer "F.Cu") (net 8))
 (segment (start 155.05 76.1) (end 155.95 75.2) (width 0.25) (layer "F.Cu") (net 8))
 (segment (start 144 71.31) (end 145.6 72.91) (width 0.25) (layer "F.Cu") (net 9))
 (segment (start 145.6 72.91) (end 145.6 74.1) (width 0.25) (layer "F.Cu") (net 9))
 (segment (start 145.6 74.1) (end 145.6 74.875) (width 0.25) (layer "F.Cu") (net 9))
 (segment (start 144 70.21) (end 144 71.31) (width 0.25) (layer "F.Cu") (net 9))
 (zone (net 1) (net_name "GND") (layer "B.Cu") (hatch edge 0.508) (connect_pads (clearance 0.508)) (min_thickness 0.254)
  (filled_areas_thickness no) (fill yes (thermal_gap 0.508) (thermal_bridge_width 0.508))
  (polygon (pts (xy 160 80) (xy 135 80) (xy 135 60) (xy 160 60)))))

